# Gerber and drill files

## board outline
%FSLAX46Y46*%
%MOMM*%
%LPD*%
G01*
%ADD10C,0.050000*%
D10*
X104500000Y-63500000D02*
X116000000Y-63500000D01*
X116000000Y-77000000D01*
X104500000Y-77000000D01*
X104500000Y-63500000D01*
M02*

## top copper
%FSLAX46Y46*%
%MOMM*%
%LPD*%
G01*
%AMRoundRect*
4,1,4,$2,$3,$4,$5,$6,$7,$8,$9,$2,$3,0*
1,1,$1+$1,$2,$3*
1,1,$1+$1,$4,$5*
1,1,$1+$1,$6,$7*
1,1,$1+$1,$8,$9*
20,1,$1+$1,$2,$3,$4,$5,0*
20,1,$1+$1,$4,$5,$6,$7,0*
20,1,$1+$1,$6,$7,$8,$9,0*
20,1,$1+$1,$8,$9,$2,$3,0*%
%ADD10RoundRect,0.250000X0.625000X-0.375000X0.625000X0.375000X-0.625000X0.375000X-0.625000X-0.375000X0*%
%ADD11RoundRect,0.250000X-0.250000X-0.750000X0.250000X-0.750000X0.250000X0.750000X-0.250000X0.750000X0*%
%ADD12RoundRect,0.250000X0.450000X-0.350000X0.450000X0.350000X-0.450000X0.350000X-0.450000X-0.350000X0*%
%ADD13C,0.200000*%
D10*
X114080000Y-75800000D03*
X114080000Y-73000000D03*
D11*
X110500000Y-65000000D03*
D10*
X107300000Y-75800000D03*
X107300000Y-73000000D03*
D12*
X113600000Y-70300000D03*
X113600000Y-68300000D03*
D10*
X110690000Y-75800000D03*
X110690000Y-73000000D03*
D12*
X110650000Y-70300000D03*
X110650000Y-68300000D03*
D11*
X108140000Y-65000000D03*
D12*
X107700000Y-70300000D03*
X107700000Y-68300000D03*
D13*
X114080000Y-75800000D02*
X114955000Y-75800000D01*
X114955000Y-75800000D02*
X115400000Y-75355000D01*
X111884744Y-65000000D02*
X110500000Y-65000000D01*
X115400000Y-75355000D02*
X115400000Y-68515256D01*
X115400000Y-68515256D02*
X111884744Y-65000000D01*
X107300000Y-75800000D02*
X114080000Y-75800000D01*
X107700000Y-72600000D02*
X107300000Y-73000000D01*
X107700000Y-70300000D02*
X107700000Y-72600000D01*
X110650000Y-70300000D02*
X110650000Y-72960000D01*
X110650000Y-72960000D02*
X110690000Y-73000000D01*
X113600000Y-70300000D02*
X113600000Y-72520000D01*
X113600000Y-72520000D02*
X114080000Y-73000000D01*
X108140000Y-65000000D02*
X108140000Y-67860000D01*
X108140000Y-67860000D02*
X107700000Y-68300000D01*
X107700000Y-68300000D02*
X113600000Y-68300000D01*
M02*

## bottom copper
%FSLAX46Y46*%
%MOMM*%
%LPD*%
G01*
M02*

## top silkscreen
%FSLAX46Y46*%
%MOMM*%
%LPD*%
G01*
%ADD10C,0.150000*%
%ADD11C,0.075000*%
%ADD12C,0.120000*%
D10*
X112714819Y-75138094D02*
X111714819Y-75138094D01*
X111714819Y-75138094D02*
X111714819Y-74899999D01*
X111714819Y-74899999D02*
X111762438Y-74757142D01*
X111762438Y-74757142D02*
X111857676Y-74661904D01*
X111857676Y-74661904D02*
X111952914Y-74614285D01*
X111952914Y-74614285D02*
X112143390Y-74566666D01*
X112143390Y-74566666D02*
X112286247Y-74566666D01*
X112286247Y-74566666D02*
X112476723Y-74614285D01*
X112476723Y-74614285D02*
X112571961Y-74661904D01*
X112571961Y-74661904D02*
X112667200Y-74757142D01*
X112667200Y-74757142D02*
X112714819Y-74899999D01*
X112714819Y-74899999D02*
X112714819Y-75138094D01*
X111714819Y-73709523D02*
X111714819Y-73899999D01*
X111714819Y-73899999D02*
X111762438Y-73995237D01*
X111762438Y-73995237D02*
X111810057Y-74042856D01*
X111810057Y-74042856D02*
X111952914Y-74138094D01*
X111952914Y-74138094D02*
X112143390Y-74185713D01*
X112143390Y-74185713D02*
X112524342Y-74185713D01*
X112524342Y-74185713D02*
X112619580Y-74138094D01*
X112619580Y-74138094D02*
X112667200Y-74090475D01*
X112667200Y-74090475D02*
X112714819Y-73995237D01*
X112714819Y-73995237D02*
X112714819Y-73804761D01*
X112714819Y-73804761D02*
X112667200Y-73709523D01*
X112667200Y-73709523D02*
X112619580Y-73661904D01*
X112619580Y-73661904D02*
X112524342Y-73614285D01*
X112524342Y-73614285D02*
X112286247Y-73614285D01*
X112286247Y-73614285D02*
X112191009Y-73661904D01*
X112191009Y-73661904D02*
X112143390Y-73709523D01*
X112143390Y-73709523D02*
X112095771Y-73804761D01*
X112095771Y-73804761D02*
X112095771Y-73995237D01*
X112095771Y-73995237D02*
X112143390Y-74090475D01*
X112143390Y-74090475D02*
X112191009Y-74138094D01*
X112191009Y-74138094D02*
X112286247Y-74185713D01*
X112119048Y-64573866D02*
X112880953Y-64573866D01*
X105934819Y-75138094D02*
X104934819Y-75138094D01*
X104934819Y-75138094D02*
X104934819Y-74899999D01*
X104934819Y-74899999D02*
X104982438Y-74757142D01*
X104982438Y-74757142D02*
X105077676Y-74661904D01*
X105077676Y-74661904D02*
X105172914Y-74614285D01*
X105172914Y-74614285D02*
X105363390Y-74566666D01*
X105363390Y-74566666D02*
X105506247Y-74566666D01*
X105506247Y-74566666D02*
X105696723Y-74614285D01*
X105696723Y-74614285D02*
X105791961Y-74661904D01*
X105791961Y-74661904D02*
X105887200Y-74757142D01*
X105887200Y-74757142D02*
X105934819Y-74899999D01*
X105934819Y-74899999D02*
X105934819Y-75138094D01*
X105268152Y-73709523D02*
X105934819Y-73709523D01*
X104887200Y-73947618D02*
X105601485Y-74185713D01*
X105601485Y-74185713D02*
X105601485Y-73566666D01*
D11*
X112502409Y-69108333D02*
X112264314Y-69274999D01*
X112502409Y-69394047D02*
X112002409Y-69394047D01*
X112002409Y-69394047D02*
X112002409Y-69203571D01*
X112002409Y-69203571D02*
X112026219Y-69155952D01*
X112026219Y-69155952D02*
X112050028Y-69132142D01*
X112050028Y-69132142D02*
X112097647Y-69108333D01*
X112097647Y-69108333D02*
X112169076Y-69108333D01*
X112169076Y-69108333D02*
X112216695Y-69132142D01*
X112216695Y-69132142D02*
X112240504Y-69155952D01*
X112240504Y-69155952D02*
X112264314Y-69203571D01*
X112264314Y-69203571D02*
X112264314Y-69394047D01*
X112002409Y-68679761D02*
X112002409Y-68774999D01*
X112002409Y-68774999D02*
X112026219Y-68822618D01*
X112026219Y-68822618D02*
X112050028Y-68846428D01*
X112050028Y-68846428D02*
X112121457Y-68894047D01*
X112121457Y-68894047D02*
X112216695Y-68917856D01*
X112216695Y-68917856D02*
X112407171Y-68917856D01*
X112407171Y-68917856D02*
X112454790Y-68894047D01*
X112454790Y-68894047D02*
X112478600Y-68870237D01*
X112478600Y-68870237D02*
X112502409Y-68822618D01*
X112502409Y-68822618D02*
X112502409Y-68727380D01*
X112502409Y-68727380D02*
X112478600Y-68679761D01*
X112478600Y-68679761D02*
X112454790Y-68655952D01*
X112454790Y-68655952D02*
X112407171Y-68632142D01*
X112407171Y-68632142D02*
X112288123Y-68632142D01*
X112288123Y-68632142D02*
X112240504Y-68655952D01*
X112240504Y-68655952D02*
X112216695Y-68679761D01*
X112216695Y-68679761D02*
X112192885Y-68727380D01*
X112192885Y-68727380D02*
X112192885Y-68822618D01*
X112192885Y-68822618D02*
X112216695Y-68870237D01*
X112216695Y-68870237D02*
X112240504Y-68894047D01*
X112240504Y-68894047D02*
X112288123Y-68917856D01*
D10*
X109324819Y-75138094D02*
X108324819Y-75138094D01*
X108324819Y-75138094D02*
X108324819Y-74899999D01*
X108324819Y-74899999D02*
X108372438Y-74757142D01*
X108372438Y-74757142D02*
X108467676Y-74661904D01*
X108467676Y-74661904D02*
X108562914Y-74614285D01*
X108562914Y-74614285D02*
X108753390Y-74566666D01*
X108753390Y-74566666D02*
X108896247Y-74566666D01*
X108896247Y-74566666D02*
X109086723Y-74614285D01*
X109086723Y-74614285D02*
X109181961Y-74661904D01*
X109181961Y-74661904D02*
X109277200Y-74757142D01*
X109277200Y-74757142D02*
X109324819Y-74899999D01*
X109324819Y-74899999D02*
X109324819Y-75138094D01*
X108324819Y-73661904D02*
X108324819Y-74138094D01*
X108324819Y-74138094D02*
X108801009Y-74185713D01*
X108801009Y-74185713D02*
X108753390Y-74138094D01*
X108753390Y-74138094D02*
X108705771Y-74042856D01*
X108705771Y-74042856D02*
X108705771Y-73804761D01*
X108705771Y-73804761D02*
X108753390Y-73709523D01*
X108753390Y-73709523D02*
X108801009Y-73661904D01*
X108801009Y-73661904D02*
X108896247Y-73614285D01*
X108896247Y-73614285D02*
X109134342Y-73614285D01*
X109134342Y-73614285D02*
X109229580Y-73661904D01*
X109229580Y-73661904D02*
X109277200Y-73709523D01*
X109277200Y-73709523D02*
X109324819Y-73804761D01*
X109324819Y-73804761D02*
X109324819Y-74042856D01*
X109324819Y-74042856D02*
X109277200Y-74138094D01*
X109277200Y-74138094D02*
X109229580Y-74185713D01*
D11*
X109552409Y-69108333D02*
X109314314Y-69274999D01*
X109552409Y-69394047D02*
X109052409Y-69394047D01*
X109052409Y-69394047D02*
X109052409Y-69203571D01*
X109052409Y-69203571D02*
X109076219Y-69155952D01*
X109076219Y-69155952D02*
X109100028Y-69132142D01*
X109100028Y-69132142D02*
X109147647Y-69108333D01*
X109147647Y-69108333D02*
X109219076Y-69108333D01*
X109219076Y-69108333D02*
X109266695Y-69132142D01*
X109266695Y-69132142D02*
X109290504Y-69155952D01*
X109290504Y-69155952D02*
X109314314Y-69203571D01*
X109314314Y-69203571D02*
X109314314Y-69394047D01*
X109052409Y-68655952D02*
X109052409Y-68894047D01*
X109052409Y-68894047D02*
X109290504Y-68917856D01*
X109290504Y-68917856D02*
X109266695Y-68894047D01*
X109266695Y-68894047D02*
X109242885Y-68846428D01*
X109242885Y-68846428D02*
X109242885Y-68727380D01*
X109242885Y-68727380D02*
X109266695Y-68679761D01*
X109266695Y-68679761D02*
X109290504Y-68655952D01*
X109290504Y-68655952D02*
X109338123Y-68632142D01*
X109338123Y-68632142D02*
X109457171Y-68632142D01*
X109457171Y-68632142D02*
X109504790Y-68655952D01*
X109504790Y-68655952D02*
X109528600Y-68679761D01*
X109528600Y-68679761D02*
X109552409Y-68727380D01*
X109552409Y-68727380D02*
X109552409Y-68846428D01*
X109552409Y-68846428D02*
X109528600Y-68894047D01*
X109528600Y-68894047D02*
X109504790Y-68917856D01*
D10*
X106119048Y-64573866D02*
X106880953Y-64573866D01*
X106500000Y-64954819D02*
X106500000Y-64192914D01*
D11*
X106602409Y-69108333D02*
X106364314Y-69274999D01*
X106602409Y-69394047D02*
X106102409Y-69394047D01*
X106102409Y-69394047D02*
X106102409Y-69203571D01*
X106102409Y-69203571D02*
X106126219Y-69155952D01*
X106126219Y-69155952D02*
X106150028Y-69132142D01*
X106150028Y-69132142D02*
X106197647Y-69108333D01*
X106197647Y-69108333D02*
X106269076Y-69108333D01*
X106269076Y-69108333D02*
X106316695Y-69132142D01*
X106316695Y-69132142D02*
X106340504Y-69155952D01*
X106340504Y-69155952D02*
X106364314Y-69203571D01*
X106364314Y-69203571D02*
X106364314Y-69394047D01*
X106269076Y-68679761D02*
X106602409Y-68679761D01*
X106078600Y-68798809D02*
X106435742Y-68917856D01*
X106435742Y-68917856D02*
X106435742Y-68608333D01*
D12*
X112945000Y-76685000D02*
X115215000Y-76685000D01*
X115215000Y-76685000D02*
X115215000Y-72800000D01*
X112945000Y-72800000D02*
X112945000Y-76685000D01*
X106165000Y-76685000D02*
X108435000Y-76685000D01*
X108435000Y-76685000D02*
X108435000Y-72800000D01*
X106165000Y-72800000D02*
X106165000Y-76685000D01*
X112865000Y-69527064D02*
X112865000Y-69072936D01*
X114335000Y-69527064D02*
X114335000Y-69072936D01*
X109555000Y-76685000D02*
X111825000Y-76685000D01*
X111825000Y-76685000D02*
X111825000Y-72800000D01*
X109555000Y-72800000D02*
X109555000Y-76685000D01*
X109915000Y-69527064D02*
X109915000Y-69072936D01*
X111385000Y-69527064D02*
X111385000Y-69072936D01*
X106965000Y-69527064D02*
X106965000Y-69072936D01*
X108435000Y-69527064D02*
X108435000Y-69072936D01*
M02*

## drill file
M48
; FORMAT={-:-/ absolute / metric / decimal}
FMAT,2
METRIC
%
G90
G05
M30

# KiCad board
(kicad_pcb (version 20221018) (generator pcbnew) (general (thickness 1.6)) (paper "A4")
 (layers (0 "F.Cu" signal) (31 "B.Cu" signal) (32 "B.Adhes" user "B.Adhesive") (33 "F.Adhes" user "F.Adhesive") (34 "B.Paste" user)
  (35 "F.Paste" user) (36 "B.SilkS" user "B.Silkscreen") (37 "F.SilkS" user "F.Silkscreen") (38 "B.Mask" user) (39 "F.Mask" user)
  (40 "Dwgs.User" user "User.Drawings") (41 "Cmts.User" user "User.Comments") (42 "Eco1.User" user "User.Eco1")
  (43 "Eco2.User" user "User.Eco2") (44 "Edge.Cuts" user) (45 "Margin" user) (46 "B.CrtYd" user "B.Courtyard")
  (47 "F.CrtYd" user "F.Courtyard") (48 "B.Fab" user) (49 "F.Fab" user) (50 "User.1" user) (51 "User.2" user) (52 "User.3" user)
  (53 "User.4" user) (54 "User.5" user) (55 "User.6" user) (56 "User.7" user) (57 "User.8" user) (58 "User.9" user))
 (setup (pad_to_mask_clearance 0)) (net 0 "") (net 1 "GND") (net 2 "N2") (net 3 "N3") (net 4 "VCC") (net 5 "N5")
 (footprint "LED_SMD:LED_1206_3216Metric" (layer "F.Cu") (at 114.08 74.4 90)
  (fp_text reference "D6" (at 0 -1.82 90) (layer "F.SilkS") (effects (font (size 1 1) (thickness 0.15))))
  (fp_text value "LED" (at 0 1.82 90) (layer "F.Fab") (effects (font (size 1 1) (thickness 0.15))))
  (fp_line (start -2.285 -1.135) (end -2.285 1.135) (stroke (width 0.12) (type solid)) (layer "F.SilkS"))
  (fp_line (start -2.285 1.135) (end 1.6 1.135) (stroke (width 0.12) (type solid)) (layer "F.SilkS"))
  (fp_line (start 1.6 -1.135) (end -2.285 -1.135) (stroke (width 0.12) (type solid)) (layer "F.SilkS"))
  (pad "1" smd roundrect (at -1.4 0 90) (size 1.25 1.75) (layers "F.Cu" "F.Paste" "F.Mask") (roundrect_rratio 0.2) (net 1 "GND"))
  (pad "2" smd roundrect (at 1.4 0 90) (size 1.25 1.75) (layers "F.Cu" "F.Paste" "F.Mask") (roundrect_rratio 0.2) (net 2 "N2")))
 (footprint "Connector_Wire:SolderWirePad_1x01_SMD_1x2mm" (layer "F.Cu") (at 110.5 65)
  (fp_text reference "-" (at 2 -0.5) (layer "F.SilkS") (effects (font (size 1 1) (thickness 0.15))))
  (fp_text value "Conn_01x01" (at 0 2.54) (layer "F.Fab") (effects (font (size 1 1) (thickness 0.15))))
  (pad "1" smd roundrect (at 0 0) (size 1 2) (layers "F.Cu" "F.Paste" "F.Mask") (roundrect_rratio 0.25) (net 1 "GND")))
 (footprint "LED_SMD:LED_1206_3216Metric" (layer "F.Cu") (at 107.3 74.4 90)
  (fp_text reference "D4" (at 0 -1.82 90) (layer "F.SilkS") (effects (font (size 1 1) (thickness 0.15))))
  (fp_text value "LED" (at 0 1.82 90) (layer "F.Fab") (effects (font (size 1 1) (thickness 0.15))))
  (fp_line (start -2.285 -1.135) (end -2.285 1.135) (stroke (width 0.12) (type solid)) (layer "F.SilkS"))
  (fp_line (start -2.285 1.135) (end 1.6 1.135) (stroke (width 0.12) (type solid)) (layer "F.SilkS"))
  (fp_line (start 1.6 -1.135) (end -2.285 -1.135) (stroke (width 0.12) (type solid)) (layer "F.SilkS"))
  (pad "1" smd roundrect (at -1.4 0 90) (size 1.25 1.75) (layers "F.Cu" "F.Paste" "F.Mask") (roundrect_rratio 0.2) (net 1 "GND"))
  (pad "2" smd roundrect (at 1.4 0 90) (size 1.25 1.75) (layers "F.Cu" "F.Paste" "F.Mask") (roundrect_rratio 0.2) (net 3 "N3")))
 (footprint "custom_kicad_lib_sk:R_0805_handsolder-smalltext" (layer "F.Cu") (at 113.6 69.3 90)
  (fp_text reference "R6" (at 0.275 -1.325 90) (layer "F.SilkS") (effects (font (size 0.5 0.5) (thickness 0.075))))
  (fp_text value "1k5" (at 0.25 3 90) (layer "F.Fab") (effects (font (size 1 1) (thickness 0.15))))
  (fp_line (start -0.227064 -0.735) (end 0.227064 -0.735) (stroke (width 0.12) (type solid)) (layer "F.SilkS"))
  (fp_line (start -0.227064 0.735) (end 0.227064 0.735) (stroke (width 0.12) (type solid)) (layer "F.SilkS"))
  (pad "1" smd roundrect (at -1 0 90) (size 1.2 1.4) (layers "F.Cu" "F.Paste" "F.Mask") (roundrect_rratio 0.2083333333) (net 2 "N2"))
  (pad "2" smd roundrect (at 1 0 90) (size 1.2 1.4) (layers "F.Cu" "F.Paste" "F.Mask") (roundrect_rratio 0.2083333333) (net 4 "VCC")))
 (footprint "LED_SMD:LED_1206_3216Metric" (layer "F.Cu") (at 110.69 74.4 90)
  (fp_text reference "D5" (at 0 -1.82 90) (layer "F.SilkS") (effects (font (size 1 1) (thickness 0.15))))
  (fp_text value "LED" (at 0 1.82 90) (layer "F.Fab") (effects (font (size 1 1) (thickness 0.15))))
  (fp_line (start -2.285 -1.135) (end -2.285 1.135) (stroke (width 0.12) (type solid)) (layer "F.SilkS"))
  (fp_line (start -2.285 1.135) (end 1.6 1.135) (stroke (width 0.12) (type solid)) (layer "F.SilkS"))
  (fp_line (start 1.6 -1.135) (end -2.285 -1.135) (stroke (width 0.12) (type solid)) (layer "F.SilkS"))
  (pad "1" smd roundrect (at -1.4 0 90) (size 1.25 1.75) (layers "F.Cu" "F.Paste" "F.Mask") (roundrect_rratio 0.2) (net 1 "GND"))
  (pad "2" smd roundrect (at 1.4 0 90) (size 1.25 1.75) (layers "F.Cu" "F.Paste" "F.Mask") (roundrect_rratio 0.2) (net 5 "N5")))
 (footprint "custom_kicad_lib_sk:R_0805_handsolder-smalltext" (layer "F.Cu") (at 110.65 69.3 90)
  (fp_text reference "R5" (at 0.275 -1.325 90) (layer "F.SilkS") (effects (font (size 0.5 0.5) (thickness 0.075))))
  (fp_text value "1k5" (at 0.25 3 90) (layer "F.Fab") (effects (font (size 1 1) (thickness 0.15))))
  (fp_line (start -0.227064 -0.735) (end 0.227064 -0.735) (stroke (width 0.12) (type solid)) (layer "F.SilkS"))
  (fp_line (start -0.227064 0.735) (end 0.227064 0.735) (stroke (width 0.12) (type solid)) (layer "F.SilkS"))
  (pad "1" smd roundrect (at -1 0 90) (size 1.2 1.4) (layers "F.Cu" "F.Paste" "F.Mask") (roundrect_rratio 0.2083333333) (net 5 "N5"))
  (pad "2" smd roundrect (at 1 0 90) (size 1.2 1.4) (layers "F.Cu" "F.Paste" "F.Mask") (roundrect_rratio 0.2083333333) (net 4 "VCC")))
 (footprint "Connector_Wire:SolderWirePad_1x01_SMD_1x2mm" (layer "F.Cu") (at 108.14 65)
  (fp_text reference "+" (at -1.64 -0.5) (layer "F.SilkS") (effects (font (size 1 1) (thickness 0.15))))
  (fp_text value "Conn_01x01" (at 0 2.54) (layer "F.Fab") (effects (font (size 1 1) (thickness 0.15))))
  (pad "1" smd roundrect (at 0 0) (size 1 2) (layers "F.Cu" "F.Paste" "F.Mask") (roundrect_rratio 0.25) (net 4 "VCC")))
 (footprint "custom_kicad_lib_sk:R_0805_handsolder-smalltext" (layer "F.Cu") (at 107.7 69.3 90)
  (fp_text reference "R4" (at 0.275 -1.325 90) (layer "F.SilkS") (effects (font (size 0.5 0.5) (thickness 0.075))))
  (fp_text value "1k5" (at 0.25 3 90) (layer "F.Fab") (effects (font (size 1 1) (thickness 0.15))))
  (fp_line (start -0.227064 -0.735) (end 0.227064 -0.735) (stroke (width 0.12) (type solid)) (layer "F.SilkS"))
  (fp_line (start -0.227064 0.735) (end 0.227064 0.735) (stroke (width 0.12) (type solid)) (layer "F.SilkS"))
  (pad "1" smd roundrect (at -1 0 90) (size 1.2 1.4) (layers "F.Cu" "F.Paste" "F.Mask") (roundrect_rratio 0.2083333333) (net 3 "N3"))
  (pad "2" smd roundrect (at 1 0 90) (size 1.2 1.4) (layers "F.Cu" "F.Paste" "F.Mask") (roundrect_rratio 0.2083333333) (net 4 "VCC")))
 (gr_rect (start 104.5 63.5) (end 116 77) (stroke (width 0.05) (type default)) (fill none) (layer "Edge.Cuts"))
 (segment (start 114.08 75.8) (end 114.955 75.8) (width 0.2) (layer "F.Cu") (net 1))
 (segment (start 114.955 75.8) (end 115.4 75.355) (width 0.2) (layer "F.Cu") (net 1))
 (segment (start 111.884744 65) (end 110.5 65) (width 0.2) (layer "F.Cu") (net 1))
 (segment (start 115.4 75.355) (end 115.4 68.515256) (width 0.2) (layer "F.Cu") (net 1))
 (segment (start 115.4 68.515256) (end 111.884744 65) (width 0.2) (layer "F.Cu") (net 1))
 (segment (start 107.3 75.8) (end 114.08 75.8) (width 0.2) (layer "F.Cu") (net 1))
 (segment (start 107.7 72.6) (end 107.3 73) (width 0.2) (layer "F.Cu") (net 3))
 (segment (start 107.7 70.3) (end 107.7 72.6) (width 0.2) (layer "F.Cu") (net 3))
 (segment (start 110.65 70.3) (end 110.65 72.96) (width 0.2) (layer "F.Cu") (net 5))
 (segment (start 110.65 72.96) (end 110.69 73) (width 0.2) (layer "F.Cu") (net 5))
 (segment (start 113.6 70.3) (end 113.6 72.52) (width 0.2) (layer "F.Cu") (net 2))
 (segment (start 113.6 72.52) (end 114.08 73) (width 0.2) (layer "F.Cu") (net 2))
 (segment (start 108.14 65) (end 108.14 67.86) (width 0.2) (layer "F.Cu") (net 4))
 (segment (start 108.14 67.86) (end 107.7 68.3) (width 0.2) (layer "F.Cu") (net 4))
 (segment (start 107.7 68.3) (end 113.6 68.3) (width 0.2) (layer "F.Cu") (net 4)))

